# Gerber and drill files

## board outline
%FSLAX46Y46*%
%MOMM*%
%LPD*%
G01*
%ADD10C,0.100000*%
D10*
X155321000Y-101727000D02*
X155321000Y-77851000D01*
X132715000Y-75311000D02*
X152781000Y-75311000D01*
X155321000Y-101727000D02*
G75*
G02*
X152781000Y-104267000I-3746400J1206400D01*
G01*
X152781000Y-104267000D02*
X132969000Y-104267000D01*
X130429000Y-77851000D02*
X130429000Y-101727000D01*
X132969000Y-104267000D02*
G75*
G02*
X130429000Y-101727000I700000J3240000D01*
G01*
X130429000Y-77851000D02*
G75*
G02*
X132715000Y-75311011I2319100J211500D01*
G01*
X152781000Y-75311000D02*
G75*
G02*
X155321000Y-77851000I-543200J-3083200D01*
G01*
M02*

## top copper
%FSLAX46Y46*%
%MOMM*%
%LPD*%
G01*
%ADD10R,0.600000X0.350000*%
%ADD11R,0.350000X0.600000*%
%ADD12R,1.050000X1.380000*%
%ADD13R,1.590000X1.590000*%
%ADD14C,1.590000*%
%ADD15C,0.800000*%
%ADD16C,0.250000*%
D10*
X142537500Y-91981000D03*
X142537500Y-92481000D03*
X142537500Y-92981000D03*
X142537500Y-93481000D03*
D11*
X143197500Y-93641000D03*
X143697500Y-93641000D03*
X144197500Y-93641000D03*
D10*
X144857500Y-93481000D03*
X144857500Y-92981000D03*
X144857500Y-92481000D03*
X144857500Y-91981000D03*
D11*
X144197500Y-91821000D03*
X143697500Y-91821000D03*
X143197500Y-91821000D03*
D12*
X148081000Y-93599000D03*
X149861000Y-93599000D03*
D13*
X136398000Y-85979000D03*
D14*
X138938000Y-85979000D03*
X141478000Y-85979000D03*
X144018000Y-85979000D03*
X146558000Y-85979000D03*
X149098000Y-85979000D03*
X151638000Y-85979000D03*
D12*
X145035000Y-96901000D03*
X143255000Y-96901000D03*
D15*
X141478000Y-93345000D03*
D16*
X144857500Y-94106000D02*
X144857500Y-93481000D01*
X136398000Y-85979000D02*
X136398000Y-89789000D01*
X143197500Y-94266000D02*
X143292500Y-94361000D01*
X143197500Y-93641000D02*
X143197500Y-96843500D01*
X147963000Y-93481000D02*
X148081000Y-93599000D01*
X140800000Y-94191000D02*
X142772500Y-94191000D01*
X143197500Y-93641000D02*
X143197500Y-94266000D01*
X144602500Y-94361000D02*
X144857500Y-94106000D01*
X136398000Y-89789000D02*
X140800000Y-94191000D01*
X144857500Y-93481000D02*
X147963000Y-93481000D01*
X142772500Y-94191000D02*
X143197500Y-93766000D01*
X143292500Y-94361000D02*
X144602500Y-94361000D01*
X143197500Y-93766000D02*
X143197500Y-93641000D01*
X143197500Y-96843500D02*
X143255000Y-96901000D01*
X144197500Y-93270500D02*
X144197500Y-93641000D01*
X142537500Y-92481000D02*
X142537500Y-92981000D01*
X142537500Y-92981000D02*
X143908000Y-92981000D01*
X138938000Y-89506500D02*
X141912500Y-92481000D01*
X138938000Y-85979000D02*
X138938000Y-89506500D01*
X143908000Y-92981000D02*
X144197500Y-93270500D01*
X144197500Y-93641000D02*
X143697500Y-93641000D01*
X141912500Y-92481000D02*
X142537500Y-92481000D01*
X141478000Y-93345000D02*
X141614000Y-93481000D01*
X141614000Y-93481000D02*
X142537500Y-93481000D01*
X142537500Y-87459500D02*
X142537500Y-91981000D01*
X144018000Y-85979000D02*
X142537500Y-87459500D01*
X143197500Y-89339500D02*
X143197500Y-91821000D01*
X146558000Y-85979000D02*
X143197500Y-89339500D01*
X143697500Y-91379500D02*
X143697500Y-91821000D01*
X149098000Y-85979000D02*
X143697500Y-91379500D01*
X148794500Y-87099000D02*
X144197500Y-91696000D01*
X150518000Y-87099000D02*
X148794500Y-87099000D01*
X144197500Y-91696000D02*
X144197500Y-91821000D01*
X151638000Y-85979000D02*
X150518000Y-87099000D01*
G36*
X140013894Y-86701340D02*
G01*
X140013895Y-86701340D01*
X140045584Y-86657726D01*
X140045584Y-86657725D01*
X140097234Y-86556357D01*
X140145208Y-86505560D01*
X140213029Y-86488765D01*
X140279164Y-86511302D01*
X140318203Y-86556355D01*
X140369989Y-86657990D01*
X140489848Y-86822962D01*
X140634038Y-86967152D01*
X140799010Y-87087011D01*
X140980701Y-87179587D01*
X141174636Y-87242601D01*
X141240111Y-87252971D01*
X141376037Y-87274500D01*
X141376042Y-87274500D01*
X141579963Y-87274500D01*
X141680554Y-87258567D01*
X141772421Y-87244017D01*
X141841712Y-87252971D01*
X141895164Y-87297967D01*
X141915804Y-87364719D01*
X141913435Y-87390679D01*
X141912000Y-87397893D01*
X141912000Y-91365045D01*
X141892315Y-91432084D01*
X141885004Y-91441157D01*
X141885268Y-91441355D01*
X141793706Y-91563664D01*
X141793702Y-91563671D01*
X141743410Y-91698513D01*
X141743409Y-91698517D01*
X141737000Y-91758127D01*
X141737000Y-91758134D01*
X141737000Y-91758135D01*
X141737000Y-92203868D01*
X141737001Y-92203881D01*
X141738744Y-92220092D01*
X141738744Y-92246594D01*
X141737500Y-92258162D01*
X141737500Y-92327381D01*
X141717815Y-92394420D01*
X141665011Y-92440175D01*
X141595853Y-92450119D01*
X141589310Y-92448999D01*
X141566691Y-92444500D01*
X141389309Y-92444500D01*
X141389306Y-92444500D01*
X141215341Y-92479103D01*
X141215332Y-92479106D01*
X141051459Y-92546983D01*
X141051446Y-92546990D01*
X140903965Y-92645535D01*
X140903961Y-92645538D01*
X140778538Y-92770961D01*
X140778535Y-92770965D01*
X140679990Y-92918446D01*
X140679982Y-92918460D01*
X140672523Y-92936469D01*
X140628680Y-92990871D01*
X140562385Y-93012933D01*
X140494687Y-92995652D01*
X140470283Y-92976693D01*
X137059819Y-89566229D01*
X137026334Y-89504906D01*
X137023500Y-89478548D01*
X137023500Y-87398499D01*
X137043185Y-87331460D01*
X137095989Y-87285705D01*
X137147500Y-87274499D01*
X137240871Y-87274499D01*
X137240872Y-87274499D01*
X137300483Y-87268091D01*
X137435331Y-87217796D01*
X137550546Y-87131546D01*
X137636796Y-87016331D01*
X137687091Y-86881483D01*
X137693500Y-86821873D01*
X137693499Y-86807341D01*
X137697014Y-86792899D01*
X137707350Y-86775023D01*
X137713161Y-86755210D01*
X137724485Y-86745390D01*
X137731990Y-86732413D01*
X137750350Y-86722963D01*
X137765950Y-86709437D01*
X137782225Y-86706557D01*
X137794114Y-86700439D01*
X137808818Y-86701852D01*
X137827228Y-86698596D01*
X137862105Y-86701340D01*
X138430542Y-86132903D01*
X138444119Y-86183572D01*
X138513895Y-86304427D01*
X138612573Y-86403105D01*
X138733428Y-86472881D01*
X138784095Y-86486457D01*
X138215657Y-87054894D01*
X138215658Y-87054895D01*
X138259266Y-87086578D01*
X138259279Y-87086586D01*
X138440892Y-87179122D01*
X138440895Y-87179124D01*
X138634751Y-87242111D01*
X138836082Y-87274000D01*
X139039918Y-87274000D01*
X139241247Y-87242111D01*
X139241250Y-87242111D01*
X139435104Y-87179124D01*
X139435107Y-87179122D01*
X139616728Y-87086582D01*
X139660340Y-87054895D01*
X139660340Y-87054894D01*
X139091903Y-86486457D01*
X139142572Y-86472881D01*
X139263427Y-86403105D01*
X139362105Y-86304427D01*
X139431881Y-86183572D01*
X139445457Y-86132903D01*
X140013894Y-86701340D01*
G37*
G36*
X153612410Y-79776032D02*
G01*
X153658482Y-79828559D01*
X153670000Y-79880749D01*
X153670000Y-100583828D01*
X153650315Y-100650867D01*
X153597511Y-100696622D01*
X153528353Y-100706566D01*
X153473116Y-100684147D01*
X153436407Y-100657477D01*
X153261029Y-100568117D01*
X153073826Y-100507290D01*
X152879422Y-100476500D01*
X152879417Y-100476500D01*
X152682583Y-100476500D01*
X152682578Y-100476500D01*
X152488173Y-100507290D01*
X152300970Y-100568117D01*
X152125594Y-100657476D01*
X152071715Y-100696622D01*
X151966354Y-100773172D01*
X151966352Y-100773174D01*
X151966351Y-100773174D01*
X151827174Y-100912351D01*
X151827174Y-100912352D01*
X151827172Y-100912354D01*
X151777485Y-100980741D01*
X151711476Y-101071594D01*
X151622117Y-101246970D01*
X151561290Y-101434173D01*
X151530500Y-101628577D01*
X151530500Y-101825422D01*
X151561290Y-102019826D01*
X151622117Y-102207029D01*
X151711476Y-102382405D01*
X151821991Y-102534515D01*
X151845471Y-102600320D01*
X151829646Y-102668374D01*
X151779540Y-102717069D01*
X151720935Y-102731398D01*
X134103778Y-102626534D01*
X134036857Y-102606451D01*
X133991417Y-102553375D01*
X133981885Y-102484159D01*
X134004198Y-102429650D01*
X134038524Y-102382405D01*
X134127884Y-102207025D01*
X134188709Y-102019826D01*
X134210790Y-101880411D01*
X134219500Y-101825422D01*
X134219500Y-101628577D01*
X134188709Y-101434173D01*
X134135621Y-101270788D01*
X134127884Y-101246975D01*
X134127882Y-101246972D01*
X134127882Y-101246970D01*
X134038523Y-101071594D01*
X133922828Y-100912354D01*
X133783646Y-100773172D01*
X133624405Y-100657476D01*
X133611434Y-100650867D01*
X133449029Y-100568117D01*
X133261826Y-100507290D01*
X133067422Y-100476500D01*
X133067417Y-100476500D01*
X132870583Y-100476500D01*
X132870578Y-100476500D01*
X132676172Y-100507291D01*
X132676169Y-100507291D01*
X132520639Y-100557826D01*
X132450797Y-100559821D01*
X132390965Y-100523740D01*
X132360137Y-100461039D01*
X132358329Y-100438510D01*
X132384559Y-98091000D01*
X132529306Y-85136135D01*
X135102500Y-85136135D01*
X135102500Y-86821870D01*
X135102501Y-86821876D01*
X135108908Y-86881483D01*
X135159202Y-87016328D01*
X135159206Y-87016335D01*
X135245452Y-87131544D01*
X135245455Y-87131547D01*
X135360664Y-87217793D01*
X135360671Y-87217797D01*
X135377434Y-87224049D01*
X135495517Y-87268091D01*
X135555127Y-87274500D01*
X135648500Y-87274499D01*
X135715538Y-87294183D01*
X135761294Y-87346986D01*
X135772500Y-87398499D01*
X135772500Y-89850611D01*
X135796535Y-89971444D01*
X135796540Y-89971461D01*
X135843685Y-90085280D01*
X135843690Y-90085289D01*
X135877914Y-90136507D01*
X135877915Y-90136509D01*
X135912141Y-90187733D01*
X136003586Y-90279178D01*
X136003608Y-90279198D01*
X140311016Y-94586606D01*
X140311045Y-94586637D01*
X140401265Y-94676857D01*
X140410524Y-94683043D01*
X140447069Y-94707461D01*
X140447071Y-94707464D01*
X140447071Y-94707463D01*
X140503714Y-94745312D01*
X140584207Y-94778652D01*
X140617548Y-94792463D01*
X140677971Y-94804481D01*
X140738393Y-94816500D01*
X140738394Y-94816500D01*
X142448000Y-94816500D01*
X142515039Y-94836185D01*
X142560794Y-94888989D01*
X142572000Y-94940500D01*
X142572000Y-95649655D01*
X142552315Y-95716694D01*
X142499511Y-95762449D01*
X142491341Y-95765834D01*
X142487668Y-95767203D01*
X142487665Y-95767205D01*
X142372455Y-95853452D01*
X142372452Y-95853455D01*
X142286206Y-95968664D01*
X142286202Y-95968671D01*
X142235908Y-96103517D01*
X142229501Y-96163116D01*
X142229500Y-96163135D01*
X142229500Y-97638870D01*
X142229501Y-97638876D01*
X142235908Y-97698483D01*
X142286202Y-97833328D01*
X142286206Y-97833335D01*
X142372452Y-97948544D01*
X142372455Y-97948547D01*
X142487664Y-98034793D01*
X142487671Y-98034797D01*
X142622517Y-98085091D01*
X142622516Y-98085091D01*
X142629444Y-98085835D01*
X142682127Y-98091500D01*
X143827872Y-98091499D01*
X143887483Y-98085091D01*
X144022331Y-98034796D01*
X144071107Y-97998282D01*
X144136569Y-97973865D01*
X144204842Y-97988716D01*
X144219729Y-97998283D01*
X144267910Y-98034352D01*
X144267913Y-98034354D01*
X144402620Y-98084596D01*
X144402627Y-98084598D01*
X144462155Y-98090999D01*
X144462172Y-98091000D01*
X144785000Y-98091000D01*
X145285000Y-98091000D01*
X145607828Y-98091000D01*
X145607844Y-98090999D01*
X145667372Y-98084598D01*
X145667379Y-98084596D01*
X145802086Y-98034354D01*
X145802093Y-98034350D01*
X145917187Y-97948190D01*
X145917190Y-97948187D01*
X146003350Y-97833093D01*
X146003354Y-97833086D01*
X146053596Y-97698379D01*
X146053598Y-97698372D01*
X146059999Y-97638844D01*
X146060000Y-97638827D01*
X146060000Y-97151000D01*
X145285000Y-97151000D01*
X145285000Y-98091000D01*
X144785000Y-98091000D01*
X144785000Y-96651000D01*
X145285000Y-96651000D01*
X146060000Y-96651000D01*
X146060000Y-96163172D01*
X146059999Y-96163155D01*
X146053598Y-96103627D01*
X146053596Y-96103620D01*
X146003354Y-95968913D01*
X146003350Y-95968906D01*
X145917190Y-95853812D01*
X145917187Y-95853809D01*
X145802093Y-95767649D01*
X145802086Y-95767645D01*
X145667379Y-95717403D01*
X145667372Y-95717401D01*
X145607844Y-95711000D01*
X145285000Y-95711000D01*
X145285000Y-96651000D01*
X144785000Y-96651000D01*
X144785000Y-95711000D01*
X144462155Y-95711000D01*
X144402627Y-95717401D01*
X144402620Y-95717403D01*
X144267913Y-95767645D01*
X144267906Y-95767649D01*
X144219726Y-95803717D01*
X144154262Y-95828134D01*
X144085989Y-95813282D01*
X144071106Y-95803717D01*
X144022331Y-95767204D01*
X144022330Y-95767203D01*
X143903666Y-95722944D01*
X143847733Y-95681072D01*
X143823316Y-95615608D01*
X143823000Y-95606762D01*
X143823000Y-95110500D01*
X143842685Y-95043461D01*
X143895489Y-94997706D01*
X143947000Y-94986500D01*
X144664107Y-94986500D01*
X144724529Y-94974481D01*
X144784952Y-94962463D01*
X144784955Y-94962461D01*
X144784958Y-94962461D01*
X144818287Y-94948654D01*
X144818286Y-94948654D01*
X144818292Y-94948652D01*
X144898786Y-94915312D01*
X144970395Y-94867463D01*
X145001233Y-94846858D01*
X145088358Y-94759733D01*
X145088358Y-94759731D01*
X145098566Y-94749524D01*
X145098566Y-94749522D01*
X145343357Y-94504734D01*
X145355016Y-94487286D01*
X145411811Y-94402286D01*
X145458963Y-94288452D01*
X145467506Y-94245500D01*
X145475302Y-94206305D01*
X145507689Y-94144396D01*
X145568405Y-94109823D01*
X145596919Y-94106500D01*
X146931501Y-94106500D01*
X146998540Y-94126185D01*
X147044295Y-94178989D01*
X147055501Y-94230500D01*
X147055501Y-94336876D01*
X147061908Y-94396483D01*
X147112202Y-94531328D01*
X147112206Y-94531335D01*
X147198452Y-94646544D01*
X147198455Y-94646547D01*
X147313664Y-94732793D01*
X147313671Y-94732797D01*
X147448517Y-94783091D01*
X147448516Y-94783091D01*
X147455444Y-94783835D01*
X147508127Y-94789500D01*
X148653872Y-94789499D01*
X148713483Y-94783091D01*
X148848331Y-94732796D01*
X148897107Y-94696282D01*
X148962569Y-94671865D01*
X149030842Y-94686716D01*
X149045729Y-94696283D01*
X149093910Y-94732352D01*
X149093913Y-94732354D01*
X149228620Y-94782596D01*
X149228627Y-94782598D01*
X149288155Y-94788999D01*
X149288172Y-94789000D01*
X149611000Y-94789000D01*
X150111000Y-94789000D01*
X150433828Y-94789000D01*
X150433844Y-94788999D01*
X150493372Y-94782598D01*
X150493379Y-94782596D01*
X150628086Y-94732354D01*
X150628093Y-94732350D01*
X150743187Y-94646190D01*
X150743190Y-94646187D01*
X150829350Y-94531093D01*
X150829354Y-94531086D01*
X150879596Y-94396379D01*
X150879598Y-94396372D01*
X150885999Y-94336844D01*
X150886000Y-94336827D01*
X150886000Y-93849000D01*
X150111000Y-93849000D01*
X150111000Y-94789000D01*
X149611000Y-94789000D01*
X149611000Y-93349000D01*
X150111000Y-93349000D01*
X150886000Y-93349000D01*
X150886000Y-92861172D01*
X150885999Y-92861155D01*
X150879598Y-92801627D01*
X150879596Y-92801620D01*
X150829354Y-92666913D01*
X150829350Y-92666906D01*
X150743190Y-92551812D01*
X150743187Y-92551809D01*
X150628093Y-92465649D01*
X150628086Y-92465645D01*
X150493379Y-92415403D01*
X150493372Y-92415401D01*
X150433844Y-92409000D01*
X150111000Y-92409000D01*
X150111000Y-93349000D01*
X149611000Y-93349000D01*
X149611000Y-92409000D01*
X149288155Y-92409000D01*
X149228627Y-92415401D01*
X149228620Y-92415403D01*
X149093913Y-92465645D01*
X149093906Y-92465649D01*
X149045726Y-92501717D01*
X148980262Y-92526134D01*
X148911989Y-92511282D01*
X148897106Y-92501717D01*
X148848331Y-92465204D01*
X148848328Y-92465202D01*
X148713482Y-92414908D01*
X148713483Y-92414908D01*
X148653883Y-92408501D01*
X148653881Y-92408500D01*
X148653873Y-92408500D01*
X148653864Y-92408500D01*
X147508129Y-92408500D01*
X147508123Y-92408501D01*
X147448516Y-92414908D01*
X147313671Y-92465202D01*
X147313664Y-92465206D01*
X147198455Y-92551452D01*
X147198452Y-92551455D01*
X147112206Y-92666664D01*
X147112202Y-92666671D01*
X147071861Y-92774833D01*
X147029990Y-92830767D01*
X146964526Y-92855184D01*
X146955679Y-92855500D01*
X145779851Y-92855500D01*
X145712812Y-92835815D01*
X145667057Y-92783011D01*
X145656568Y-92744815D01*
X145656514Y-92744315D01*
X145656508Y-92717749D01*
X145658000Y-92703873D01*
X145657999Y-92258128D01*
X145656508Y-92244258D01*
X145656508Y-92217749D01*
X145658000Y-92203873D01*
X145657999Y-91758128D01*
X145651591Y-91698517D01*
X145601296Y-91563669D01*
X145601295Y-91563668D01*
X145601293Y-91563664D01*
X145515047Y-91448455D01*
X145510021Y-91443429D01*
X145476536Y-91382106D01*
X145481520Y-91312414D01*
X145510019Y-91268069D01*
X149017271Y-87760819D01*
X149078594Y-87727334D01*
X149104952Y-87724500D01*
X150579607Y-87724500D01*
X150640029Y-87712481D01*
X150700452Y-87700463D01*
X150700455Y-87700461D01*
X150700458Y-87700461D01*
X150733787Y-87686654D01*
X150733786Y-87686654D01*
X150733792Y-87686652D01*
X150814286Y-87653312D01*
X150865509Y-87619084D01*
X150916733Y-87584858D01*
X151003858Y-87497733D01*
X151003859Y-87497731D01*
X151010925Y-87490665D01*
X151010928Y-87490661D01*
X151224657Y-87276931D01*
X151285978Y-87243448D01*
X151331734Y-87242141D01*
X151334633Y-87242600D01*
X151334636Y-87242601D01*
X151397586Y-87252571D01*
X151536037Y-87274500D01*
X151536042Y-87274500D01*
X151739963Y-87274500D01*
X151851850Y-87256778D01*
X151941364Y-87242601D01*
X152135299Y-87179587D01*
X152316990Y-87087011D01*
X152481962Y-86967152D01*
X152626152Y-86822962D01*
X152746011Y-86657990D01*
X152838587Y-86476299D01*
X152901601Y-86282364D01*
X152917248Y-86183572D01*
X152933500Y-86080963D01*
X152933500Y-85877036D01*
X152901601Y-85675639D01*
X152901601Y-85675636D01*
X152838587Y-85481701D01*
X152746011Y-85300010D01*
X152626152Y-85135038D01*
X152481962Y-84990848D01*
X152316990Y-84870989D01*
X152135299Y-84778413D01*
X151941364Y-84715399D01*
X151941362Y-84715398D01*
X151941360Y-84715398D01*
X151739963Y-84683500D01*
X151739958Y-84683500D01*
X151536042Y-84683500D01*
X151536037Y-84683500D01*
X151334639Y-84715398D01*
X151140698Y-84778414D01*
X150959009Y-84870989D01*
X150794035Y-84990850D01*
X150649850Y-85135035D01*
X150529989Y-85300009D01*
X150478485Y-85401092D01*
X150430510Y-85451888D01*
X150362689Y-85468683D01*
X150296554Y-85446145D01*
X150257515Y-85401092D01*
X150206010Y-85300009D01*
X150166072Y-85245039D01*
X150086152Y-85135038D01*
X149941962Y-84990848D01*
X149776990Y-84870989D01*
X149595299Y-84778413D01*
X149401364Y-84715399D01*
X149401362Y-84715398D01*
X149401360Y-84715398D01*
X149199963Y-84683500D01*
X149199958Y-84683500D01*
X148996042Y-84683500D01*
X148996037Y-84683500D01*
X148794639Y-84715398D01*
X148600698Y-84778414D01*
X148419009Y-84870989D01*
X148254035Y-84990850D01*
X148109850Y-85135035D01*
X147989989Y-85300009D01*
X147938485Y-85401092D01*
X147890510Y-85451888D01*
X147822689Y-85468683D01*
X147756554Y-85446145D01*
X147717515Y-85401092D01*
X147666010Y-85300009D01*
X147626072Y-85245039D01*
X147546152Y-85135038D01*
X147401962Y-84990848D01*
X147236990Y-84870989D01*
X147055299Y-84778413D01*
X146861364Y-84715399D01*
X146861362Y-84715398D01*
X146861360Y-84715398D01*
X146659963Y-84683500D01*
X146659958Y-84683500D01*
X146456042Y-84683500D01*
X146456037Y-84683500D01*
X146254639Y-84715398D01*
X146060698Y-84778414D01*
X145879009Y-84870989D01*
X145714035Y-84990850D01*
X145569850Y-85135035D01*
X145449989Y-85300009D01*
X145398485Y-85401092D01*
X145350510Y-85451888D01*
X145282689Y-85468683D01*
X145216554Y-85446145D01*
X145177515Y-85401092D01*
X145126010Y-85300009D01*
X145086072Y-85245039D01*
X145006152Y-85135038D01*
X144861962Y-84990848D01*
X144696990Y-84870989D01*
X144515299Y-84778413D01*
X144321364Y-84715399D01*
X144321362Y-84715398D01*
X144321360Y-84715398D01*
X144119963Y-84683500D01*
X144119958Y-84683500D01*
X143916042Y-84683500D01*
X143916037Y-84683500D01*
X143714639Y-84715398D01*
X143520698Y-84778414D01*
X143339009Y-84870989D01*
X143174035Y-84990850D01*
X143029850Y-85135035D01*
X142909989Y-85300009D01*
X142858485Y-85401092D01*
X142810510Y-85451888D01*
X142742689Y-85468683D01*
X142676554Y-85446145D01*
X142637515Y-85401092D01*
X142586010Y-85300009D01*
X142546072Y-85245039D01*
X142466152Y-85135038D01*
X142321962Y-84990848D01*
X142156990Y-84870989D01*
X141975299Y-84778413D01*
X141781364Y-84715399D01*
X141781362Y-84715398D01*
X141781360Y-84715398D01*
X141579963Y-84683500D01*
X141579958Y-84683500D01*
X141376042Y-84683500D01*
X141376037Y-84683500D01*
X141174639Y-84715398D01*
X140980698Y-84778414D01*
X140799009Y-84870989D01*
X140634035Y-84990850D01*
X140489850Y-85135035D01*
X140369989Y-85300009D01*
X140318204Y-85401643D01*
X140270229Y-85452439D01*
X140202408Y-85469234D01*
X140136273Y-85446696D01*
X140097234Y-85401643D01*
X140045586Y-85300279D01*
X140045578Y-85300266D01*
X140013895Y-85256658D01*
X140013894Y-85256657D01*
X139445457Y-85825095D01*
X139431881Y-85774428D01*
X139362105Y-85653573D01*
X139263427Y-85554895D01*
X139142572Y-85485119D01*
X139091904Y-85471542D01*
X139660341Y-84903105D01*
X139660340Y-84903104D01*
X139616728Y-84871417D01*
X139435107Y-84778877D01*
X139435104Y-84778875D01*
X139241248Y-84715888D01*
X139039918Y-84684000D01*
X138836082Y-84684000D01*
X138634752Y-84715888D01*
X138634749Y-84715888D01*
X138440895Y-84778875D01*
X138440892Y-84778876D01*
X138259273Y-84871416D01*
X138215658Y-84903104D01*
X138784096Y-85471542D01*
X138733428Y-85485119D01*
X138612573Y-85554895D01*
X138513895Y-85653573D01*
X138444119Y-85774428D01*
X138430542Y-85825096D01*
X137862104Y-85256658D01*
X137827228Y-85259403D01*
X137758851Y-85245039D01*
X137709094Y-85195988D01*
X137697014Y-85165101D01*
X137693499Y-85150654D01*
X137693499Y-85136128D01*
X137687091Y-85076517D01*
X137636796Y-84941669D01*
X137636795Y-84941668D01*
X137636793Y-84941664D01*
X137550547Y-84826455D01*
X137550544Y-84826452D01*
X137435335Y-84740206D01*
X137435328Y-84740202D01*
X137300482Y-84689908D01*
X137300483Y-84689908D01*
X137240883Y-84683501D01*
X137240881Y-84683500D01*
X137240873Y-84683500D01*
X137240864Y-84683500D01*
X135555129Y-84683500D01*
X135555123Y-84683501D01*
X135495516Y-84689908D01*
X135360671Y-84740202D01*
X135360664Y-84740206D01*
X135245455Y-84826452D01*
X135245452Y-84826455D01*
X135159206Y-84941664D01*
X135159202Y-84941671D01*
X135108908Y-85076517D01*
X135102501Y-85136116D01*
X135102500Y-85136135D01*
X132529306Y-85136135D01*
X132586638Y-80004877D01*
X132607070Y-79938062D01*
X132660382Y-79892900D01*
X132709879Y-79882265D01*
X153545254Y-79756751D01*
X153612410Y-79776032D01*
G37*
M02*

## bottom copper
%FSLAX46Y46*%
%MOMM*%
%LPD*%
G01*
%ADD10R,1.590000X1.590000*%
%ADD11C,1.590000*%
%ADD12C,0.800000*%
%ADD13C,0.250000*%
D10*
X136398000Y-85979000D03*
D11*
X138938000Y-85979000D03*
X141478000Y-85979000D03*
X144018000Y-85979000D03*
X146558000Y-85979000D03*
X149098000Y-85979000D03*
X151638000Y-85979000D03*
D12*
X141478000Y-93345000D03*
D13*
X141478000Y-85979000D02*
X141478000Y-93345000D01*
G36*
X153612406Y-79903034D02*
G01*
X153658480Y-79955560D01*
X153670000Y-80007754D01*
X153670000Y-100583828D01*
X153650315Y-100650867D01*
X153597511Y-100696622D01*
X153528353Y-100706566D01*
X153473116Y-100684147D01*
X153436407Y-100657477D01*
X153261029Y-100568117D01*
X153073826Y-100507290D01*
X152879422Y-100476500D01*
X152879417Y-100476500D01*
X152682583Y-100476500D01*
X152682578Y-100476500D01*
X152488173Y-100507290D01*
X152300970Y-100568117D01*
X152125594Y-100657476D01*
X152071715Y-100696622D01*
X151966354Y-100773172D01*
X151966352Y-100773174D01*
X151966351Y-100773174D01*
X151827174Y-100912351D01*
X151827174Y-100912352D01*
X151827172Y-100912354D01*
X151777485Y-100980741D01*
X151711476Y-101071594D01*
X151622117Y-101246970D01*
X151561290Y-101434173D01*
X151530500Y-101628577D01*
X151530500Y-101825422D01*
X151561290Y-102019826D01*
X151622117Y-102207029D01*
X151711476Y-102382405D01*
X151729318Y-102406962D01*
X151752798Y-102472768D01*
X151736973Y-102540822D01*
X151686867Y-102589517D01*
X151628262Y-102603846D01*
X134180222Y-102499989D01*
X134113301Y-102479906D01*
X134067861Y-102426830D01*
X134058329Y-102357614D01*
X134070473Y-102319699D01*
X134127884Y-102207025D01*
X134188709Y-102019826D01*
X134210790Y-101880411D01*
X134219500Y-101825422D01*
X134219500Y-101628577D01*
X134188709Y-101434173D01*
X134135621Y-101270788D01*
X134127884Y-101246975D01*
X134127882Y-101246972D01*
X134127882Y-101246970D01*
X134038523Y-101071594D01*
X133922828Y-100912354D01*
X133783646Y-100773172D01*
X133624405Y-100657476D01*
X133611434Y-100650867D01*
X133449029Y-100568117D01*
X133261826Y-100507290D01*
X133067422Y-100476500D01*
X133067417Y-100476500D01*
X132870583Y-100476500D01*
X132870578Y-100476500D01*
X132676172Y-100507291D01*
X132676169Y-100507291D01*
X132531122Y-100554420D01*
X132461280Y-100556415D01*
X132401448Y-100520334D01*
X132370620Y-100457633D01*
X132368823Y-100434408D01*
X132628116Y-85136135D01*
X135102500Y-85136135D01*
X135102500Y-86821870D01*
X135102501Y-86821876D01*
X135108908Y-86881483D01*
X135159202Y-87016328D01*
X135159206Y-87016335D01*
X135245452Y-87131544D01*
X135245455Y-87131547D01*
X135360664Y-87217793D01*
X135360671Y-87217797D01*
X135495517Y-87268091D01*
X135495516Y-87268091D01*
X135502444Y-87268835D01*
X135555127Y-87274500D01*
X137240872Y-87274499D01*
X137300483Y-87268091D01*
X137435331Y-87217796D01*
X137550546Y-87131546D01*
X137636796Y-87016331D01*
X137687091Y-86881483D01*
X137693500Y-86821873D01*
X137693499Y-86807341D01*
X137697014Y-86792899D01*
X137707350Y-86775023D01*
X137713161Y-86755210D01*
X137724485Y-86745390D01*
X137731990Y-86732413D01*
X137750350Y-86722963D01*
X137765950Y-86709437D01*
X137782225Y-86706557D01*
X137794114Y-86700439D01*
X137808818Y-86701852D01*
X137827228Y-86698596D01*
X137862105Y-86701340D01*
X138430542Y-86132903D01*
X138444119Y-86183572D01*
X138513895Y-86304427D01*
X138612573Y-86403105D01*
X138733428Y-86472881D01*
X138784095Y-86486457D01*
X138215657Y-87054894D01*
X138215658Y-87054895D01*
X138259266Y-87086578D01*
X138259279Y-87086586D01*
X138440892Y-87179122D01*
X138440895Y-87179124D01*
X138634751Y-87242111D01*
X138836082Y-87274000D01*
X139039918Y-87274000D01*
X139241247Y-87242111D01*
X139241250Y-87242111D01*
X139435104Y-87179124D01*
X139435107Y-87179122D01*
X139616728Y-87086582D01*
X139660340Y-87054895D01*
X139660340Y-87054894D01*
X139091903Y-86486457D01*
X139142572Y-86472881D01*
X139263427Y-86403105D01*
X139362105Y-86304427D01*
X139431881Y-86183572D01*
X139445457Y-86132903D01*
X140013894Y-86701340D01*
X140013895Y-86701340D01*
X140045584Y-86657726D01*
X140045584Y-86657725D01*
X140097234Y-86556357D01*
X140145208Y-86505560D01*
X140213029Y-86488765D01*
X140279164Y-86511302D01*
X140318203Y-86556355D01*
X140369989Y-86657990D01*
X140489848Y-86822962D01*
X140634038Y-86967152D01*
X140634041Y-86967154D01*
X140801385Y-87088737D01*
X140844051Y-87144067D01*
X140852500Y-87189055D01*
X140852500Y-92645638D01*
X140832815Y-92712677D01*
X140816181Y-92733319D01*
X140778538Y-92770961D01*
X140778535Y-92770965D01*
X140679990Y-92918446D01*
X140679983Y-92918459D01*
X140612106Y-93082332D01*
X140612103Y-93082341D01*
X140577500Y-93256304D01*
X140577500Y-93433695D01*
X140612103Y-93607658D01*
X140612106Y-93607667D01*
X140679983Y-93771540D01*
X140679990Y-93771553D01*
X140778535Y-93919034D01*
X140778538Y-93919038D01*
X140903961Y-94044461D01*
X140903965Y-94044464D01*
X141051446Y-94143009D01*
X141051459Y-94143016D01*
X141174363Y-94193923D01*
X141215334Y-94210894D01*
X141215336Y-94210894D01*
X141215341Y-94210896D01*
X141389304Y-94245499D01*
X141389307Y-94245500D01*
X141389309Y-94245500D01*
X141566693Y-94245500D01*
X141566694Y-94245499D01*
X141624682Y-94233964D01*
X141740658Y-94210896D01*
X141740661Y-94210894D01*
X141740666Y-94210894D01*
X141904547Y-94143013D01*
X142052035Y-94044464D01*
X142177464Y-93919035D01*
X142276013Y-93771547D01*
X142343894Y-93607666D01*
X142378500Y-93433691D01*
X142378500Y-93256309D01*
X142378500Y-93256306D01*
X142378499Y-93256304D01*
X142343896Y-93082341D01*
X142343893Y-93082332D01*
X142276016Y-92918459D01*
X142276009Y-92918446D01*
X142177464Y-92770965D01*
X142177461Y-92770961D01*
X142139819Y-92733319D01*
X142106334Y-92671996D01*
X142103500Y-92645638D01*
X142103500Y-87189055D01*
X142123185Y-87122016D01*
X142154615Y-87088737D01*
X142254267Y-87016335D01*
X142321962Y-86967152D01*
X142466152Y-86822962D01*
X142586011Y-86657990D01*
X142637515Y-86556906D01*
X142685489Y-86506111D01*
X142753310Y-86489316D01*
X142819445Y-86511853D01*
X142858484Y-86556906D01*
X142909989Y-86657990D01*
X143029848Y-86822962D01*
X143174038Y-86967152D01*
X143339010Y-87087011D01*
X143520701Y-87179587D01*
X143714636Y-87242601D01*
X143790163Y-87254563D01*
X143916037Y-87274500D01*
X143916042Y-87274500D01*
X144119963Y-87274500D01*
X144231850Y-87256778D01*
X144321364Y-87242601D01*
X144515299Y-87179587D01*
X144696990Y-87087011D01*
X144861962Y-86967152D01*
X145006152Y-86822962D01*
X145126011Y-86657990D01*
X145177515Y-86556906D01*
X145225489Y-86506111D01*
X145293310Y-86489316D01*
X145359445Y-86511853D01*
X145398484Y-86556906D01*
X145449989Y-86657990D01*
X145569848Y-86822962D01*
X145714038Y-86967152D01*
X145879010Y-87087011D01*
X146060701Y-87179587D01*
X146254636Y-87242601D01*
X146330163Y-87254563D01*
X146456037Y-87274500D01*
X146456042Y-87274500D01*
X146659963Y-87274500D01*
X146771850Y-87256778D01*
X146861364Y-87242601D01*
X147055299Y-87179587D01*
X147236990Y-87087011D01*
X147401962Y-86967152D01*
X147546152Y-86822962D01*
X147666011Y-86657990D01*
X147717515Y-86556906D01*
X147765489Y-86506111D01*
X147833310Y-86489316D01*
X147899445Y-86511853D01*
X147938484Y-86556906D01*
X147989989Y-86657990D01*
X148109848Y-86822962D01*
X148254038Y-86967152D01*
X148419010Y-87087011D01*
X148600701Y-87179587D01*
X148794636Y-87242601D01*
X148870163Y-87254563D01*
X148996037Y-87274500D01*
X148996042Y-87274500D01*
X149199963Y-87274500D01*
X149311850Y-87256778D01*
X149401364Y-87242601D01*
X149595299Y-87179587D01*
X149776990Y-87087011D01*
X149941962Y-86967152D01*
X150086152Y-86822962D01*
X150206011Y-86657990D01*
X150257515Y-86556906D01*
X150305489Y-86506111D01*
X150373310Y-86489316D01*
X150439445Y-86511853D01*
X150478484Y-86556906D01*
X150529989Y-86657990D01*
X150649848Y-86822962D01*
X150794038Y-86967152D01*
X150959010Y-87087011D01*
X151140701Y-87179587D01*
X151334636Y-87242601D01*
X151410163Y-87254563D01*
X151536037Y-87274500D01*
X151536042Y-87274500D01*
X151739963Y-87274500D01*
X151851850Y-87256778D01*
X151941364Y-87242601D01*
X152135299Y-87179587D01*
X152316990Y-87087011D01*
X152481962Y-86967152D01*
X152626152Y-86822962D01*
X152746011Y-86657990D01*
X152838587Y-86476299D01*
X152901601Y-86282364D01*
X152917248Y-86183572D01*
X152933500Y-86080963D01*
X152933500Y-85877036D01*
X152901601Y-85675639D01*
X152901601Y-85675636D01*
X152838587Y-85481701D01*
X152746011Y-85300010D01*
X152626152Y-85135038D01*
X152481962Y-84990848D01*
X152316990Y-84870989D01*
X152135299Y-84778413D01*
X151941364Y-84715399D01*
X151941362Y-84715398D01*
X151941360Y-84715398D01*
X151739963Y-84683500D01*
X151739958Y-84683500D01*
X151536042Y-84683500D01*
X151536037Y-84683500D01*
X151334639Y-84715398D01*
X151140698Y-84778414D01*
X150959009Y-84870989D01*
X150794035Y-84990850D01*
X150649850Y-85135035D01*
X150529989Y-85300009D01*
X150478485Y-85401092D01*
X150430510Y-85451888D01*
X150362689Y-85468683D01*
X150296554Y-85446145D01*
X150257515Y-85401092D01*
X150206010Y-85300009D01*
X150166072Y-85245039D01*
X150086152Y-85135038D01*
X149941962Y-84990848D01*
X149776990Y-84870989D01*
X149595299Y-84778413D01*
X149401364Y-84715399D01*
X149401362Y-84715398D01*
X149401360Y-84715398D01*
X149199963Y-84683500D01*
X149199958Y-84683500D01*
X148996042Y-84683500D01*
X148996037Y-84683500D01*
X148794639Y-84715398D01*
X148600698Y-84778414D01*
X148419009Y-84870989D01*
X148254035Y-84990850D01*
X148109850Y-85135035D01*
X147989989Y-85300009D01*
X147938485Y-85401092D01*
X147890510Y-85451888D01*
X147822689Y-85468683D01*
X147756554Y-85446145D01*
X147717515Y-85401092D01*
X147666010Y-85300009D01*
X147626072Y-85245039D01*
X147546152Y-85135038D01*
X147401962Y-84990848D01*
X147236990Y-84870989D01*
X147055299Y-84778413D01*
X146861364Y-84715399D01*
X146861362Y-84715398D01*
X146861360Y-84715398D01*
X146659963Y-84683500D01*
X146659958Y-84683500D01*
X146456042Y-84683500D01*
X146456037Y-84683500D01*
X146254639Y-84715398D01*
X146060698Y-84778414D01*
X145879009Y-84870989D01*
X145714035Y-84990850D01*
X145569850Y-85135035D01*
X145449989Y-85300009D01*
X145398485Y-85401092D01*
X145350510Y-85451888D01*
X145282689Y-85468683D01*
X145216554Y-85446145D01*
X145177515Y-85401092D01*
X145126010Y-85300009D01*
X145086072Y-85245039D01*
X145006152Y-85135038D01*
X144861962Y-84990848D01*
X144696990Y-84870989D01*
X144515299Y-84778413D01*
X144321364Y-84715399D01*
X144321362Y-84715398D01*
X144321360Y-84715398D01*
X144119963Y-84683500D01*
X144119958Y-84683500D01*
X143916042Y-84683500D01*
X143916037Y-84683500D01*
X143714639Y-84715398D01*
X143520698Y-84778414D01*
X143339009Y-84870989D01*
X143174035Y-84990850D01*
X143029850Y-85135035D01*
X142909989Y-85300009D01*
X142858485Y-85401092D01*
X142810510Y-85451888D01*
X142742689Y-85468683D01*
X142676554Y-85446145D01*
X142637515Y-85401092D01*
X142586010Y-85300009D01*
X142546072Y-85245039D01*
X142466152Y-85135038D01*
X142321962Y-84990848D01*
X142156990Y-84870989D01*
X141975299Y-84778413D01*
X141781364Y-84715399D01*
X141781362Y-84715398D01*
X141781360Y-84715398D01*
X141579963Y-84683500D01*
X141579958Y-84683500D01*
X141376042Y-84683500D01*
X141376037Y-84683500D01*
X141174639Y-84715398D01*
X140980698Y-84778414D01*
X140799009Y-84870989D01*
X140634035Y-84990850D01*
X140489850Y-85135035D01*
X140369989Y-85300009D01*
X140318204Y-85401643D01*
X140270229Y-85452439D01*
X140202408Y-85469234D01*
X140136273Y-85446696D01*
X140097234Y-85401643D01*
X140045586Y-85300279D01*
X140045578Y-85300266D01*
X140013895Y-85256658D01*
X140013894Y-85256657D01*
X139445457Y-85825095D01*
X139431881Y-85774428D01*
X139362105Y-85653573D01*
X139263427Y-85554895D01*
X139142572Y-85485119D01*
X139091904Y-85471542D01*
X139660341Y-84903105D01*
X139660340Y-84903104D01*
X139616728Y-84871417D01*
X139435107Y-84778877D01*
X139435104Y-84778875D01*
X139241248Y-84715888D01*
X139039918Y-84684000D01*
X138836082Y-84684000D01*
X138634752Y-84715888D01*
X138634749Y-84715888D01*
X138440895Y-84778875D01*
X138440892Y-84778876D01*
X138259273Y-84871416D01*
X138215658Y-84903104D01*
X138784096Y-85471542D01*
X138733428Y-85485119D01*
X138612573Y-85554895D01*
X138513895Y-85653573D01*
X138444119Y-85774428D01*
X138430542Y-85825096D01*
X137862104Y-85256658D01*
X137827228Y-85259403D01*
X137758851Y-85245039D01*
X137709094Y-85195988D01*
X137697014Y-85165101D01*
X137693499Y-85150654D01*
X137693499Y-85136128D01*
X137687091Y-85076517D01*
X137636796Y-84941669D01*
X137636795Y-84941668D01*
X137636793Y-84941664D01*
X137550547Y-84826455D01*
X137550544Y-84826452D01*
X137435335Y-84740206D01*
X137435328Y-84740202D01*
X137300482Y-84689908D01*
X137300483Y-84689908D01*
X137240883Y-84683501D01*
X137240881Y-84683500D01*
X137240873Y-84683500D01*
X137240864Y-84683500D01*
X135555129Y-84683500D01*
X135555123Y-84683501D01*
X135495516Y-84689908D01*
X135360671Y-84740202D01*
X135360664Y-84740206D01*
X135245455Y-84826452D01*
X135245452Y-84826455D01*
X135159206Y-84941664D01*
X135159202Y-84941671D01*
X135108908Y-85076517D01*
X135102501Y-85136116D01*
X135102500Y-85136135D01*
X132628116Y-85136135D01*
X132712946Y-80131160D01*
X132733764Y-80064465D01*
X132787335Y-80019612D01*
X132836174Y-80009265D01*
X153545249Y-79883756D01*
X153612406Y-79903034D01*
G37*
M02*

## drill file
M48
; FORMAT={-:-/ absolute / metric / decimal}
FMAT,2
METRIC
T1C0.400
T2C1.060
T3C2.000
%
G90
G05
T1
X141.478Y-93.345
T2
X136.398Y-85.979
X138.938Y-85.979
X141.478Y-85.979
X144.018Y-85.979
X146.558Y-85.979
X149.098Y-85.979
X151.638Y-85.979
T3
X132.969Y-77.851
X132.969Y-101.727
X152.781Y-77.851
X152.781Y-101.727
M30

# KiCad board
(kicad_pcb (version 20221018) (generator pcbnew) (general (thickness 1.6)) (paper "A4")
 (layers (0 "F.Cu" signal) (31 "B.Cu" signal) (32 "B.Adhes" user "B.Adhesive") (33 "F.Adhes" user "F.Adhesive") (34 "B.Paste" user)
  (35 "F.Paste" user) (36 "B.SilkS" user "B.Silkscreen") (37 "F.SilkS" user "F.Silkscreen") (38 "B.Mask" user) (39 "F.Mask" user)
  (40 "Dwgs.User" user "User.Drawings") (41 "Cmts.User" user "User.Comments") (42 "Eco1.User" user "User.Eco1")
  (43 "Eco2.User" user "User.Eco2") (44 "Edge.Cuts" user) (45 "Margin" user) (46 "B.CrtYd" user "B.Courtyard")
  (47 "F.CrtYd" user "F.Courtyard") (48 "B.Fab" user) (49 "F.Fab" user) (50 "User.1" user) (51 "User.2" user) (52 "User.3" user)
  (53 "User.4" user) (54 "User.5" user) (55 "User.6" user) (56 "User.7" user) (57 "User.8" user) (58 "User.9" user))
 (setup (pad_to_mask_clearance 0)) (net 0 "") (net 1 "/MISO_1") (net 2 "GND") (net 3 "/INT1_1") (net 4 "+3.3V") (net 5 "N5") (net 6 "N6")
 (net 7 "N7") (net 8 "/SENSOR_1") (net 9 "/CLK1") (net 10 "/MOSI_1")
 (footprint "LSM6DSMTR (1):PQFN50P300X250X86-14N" (layer "F.Cu") (at 143.6975 92.731)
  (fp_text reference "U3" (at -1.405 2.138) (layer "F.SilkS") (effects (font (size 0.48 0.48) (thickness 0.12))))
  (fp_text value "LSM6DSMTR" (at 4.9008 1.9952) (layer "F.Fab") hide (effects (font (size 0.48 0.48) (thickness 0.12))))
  (pad "1" smd rect (at -1.16 -0.75) (size 0.6 0.35) (layers "F.Cu" "F.Paste" "F.Mask") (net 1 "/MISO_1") (solder_mask_margin 0.102))
  (pad "2" smd rect (at -1.16 -0.25) (size 0.6 0.35) (layers "F.Cu" "F.Paste" "F.Mask") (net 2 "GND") (solder_mask_margin 0.102))
  (pad "3" smd rect (at -1.16 0.25) (size 0.6 0.35) (layers "F.Cu" "F.Paste" "F.Mask") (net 2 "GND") (solder_mask_margin 0.102))
  (pad "4" smd rect (at -1.16 0.75) (size 0.6 0.35) (layers "F.Cu" "F.Paste" "F.Mask") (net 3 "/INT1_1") (solder_mask_margin 0.102))
  (pad "5" smd rect (at -0.5 0.91 90) (size 0.6 0.35) (layers "F.Cu" "F.Paste" "F.Mask") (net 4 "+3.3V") (solder_mask_margin 0.102))
  (pad "6" smd rect (at 0 0.91 90) (size 0.6 0.35) (layers "F.Cu" "F.Paste" "F.Mask") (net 2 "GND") (solder_mask_margin 0.102))
  (pad "7" smd rect (at 0.5 0.91 90) (size 0.6 0.35) (layers "F.Cu" "F.Paste" "F.Mask") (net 2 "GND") (solder_mask_margin 0.102))
  (pad "8" smd rect (at 1.16 0.75) (size 0.6 0.35) (layers "F.Cu" "F.Paste" "F.Mask") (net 4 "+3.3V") (solder_mask_margin 0.102))
  (pad "9" smd rect (at 1.16 0.25) (size 0.6 0.35) (layers "F.Cu" "F.Paste" "F.Mask") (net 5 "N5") (solder_mask_margin 0.102))
  (pad "10" smd rect (at 1.16 -0.25) (size 0.6 0.35) (layers "F.Cu" "F.Paste" "F.Mask") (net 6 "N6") (solder_mask_margin 0.102))
  (pad "11" smd rect (at 1.16 -0.75) (size 0.6 0.35) (layers "F.Cu" "F.Paste" "F.Mask") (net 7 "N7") (solder_mask_margin 0.102))
  (pad "12" smd rect (at 0.5 -0.91 90) (size 0.6 0.35) (layers "F.Cu" "F.Paste" "F.Mask") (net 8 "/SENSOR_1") (solder_mask_margin 0.102))
  (pad "13" smd rect (at 0 -0.91 90) (size 0.6 0.35) (layers "F.Cu" "F.Paste" "F.Mask") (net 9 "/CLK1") (solder_mask_margin 0.102))
  (pad "14" smd rect (at -0.5 -0.91 90) (size 0.6 0.35) (layers "F.Cu" "F.Paste" "F.Mask") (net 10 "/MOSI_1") (solder_mask_margin 0.102)))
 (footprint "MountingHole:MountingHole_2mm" (layer "F.Cu") (at 132.969 77.851)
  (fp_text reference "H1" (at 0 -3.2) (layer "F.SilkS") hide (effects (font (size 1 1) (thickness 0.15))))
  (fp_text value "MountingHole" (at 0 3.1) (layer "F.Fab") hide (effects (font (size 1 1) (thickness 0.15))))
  (pad "" np_thru_hole circle (at 0 0) (size 2 2) (drill 2) (layers "*.Cu" "*.Mask")))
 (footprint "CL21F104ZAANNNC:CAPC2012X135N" (layer "F.Cu") (at 148.971 93.599)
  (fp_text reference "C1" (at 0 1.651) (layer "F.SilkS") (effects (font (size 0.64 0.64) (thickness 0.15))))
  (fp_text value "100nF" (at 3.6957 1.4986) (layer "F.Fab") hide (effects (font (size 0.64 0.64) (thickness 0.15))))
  (pad "1" smd rect (at -0.89 0) (size 1.05 1.38) (layers "F.Cu" "F.Paste" "F.Mask") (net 4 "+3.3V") (solder_mask_margin 0.102))
  (pad "2" smd rect (at 0.89 0) (size 1.05 1.38) (layers "F.Cu" "F.Paste" "F.Mask") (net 2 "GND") (solder_mask_margin 0.102)))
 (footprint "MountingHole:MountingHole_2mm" (layer "F.Cu") (at 152.781 77.851)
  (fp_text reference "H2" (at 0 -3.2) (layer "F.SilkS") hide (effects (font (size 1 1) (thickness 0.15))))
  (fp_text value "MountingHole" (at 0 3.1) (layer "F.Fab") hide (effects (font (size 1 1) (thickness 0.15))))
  (pad "" np_thru_hole circle (at 0 0) (size 2 2) (drill 2) (layers "*.Cu" "*.Mask")))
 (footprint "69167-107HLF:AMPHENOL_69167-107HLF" (layer "F.Cu") (at 144.018 85.979)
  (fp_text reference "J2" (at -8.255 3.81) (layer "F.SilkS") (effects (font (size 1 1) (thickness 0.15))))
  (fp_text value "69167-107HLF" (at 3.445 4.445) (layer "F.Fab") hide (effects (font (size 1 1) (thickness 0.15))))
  (pad "01" thru_hole rect (at -7.62 0) (size 1.59 1.59) (drill 1.06) (layers "*.Cu" "*.Mask") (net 4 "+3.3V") (solder_mask_margin 0.102))
  (pad "02" thru_hole circle (at -5.08 0) (size 1.59 1.59) (drill 1.06) (layers "*.Cu" "*.Mask") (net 2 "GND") (solder_mask_margin 0.102))
  (pad "03" thru_hole circle (at -2.54 0) (size 1.59 1.59) (drill 1.06) (layers "*.Cu" "*.Mask") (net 3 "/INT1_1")
   (solder_mask_margin 0.102))
  (pad "04" thru_hole circle (at 0 0) (size 1.59 1.59) (drill 1.06) (layers "*.Cu" "*.Mask") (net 1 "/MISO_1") (solder_mask_margin 0.102))
  (pad "05" thru_hole circle (at 2.54 0) (size 1.59 1.59) (drill 1.06) (layers "*.Cu" "*.Mask") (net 10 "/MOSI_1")
   (solder_mask_margin 0.102))
  (pad "06" thru_hole circle (at 5.08 0) (size 1.59 1.59) (drill 1.06) (layers "*.Cu" "*.Mask") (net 9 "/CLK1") (solder_mask_margin 0.102))
  (pad "07" thru_hole circle (at 7.62 0) (size 1.59 1.59) (drill 1.06) (layers "*.Cu" "*.Mask") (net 8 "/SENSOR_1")
   (solder_mask_margin 0.102)))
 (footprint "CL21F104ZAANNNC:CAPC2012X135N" (layer "F.Cu") (at 144.145 96.901 180)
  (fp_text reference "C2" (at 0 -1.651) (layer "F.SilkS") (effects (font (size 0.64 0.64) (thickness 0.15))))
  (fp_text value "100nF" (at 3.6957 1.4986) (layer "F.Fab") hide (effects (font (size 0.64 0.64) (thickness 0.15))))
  (pad "1" smd rect (at -0.89 0 180) (size 1.05 1.38) (layers "F.Cu" "F.Paste" "F.Mask") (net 2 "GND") (solder_mask_margin 0.102))
  (pad "2" smd rect (at 0.89 0 180) (size 1.05 1.38) (layers "F.Cu" "F.Paste" "F.Mask") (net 4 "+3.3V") (solder_mask_margin 0.102)))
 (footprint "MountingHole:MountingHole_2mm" (layer "F.Cu") (at 152.781 101.727)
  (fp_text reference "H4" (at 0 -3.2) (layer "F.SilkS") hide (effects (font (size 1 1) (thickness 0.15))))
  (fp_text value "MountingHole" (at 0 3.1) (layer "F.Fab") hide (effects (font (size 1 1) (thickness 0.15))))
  (pad "" np_thru_hole circle (at 0 0) (size 2 2) (drill 2) (layers "*.Cu" "*.Mask")))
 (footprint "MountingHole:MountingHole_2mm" (layer "F.Cu") (at 132.969 101.727)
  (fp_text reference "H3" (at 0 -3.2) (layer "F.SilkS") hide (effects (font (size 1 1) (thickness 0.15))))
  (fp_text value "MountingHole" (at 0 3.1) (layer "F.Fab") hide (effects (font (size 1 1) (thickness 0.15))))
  (pad "" np_thru_hole circle (at 0 0) (size 2 2) (drill 2) (layers "*.Cu" "*.Mask")))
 (gr_line (start 155.321 101.727) (end 155.321 77.851) (stroke (width 0.1) (type default)) (layer "Edge.Cuts"))
 (gr_line (start 132.715 75.311) (end 152.781 75.311) (stroke (width 0.1) (type default)) (layer "Edge.Cuts"))
 (gr_arc (start 155.321 101.727) (mid 154.357666 103.303666) (end 152.781 104.267) (stroke (width 0.1) (type default)) (layer "Edge.Cuts"))
 (gr_line (start 152.781 104.267) (end 132.969 104.267) (stroke (width 0.1) (type default)) (layer "Edge.Cuts"))
 (gr_line (start 130.429 77.851) (end 130.429 101.727) (stroke (width 0.1) (type default)) (layer "Edge.Cuts"))
 (gr_arc (start 132.969 104.267) (mid 131.325114 103.370886) (end 130.429 101.727) (stroke (width 0.1) (type default)) (layer "Edge.Cuts"))
 (gr_arc (start 130.429 77.851) (mid 131.017178 76.08166) (end 132.715 75.311) (stroke (width 0.1) (type default)) (layer "Edge.Cuts"))
 (gr_arc (start 152.781 75.311) (mid 154.451529 76.180471) (end 155.321 77.851) (stroke (width 0.1) (type default)) (layer "Edge.Cuts"))
 (segment (start 144.8575 94.106) (end 144.8575 93.481) (width 0.25) (layer "F.Cu") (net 4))
 (segment (start 136.398 85.979) (end 136.398 89.789) (width 0.25) (layer "F.Cu") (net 4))
 (segment (start 143.1975 94.266) (end 143.2925 94.361) (width 0.25) (layer "F.Cu") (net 4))
 (segment (start 143.1975 93.641) (end 143.1975 96.8435) (width 0.25) (layer "F.Cu") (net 4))
 (segment (start 147.963 93.481) (end 148.081 93.599) (width 0.25) (layer "F.Cu") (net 4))
 (segment (start 140.8 94.191) (end 142.7725 94.191) (width 0.25) (layer "F.Cu") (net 4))
 (segment (start 143.1975 93.641) (end 143.1975 94.266) (width 0.25) (layer "F.Cu") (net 4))
 (segment (start 144.6025 94.361) (end 144.8575 94.106) (width 0.25) (layer "F.Cu") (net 4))
 (segment (start 136.398 89.789) (end 140.8 94.191) (width 0.25) (layer "F.Cu") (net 4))
 (segment (start 144.8575 93.481) (end 147.963 93.481) (width 0.25) (layer "F.Cu") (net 4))
 (segment (start 142.7725 94.191) (end 143.1975 93.766) (width 0.25) (layer "F.Cu") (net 4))
 (segment (start 143.2925 94.361) (end 144.6025 94.361) (width 0.25) (layer "F.Cu") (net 4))
 (segment (start 143.1975 93.766) (end 143.1975 93.641) (width 0.25) (layer "F.Cu") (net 4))
 (segment (start 143.1975 96.8435) (end 143.255 96.901) (width 0.25) (layer "F.Cu") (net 4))
 (segment (start 144.1975 93.2705) (end 144.1975 93.641) (width 0.25) (layer "F.Cu") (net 2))
 (segment (start 142.5375 92.481) (end 142.5375 92.981) (width 0.25) (layer "F.Cu") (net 2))
 (segment (start 142.5375 92.981) (end 143.908 92.981) (width 0.25) (layer "F.Cu") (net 2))
 (segment (start 138.938 89.5065) (end 141.9125 92.481) (width 0.25) (layer "F.Cu") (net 2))
 (segment (start 138.938 85.979) (end 138.938 89.5065) (width 0.25) (layer "F.Cu") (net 2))
 (segment (start 143.908 92.981) (end 144.1975 93.2705) (width 0.25) (layer "F.Cu") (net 2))
 (segment (start 144.1975 93.641) (end 143.6975 93.641) (width 0.25) (layer "F.Cu") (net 2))
 (segment (start 141.9125 92.481) (end 142.5375 92.481) (width 0.25) (layer "F.Cu") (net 2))
 (segment (start 141.478 93.345) (end 141.614 93.481) (width 0.25) (layer "F.Cu") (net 3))
 (segment (start 141.614 93.481) (end 142.5375 93.481) (width 0.25) (layer "F.Cu") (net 3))
 (via (at 141.478 93.345) (size 0.8) (drill 0.4) (layers "F.Cu" "B.Cu") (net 3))
 (segment (start 141.478 85.979) (end 141.478 93.345) (width 0.25) (layer "B.Cu") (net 3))
 (segment (start 142.5375 87.4595) (end 142.5375 91.981) (width 0.25) (layer "F.Cu") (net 1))
 (segment (start 144.018 85.979) (end 142.5375 87.4595) (width 0.25) (layer "F.Cu") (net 1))
 (segment (start 143.1975 89.3395) (end 143.1975 91.821) (width 0.25) (layer "F.Cu") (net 10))
 (segment (start 146.558 85.979) (end 143.1975 89.3395) (width 0.25) (layer "F.Cu") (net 10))
 (segment (start 143.6975 91.3795) (end 143.6975 91.821) (width 0.25) (layer "F.Cu") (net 9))
 (segment (start 149.098 85.979) (end 143.6975 91.3795) (width 0.25) (layer "F.Cu") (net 9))
 (segment (start 148.7945 87.099) (end 144.1975 91.696) (width 0.25) (layer "F.Cu") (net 8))
 (segment (start 150.518 87.099) (end 148.7945 87.099) (width 0.25) (layer "F.Cu") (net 8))
 (segment (start 144.1975 91.696) (end 144.1975 91.821) (width 0.25) (layer "F.Cu") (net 8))
 (segment (start 151.638 85.979) (end 150.518 87.099) (width 0.25) (layer "F.Cu") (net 8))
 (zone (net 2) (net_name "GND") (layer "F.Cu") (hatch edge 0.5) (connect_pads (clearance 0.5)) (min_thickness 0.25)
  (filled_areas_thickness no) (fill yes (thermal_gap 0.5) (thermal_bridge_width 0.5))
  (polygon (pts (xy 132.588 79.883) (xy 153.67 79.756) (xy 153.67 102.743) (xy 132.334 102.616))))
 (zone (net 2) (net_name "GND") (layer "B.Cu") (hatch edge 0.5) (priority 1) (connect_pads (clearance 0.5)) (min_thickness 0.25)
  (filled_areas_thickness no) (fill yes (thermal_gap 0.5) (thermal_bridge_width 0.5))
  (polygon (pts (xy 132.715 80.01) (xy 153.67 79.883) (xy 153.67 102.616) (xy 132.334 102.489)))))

